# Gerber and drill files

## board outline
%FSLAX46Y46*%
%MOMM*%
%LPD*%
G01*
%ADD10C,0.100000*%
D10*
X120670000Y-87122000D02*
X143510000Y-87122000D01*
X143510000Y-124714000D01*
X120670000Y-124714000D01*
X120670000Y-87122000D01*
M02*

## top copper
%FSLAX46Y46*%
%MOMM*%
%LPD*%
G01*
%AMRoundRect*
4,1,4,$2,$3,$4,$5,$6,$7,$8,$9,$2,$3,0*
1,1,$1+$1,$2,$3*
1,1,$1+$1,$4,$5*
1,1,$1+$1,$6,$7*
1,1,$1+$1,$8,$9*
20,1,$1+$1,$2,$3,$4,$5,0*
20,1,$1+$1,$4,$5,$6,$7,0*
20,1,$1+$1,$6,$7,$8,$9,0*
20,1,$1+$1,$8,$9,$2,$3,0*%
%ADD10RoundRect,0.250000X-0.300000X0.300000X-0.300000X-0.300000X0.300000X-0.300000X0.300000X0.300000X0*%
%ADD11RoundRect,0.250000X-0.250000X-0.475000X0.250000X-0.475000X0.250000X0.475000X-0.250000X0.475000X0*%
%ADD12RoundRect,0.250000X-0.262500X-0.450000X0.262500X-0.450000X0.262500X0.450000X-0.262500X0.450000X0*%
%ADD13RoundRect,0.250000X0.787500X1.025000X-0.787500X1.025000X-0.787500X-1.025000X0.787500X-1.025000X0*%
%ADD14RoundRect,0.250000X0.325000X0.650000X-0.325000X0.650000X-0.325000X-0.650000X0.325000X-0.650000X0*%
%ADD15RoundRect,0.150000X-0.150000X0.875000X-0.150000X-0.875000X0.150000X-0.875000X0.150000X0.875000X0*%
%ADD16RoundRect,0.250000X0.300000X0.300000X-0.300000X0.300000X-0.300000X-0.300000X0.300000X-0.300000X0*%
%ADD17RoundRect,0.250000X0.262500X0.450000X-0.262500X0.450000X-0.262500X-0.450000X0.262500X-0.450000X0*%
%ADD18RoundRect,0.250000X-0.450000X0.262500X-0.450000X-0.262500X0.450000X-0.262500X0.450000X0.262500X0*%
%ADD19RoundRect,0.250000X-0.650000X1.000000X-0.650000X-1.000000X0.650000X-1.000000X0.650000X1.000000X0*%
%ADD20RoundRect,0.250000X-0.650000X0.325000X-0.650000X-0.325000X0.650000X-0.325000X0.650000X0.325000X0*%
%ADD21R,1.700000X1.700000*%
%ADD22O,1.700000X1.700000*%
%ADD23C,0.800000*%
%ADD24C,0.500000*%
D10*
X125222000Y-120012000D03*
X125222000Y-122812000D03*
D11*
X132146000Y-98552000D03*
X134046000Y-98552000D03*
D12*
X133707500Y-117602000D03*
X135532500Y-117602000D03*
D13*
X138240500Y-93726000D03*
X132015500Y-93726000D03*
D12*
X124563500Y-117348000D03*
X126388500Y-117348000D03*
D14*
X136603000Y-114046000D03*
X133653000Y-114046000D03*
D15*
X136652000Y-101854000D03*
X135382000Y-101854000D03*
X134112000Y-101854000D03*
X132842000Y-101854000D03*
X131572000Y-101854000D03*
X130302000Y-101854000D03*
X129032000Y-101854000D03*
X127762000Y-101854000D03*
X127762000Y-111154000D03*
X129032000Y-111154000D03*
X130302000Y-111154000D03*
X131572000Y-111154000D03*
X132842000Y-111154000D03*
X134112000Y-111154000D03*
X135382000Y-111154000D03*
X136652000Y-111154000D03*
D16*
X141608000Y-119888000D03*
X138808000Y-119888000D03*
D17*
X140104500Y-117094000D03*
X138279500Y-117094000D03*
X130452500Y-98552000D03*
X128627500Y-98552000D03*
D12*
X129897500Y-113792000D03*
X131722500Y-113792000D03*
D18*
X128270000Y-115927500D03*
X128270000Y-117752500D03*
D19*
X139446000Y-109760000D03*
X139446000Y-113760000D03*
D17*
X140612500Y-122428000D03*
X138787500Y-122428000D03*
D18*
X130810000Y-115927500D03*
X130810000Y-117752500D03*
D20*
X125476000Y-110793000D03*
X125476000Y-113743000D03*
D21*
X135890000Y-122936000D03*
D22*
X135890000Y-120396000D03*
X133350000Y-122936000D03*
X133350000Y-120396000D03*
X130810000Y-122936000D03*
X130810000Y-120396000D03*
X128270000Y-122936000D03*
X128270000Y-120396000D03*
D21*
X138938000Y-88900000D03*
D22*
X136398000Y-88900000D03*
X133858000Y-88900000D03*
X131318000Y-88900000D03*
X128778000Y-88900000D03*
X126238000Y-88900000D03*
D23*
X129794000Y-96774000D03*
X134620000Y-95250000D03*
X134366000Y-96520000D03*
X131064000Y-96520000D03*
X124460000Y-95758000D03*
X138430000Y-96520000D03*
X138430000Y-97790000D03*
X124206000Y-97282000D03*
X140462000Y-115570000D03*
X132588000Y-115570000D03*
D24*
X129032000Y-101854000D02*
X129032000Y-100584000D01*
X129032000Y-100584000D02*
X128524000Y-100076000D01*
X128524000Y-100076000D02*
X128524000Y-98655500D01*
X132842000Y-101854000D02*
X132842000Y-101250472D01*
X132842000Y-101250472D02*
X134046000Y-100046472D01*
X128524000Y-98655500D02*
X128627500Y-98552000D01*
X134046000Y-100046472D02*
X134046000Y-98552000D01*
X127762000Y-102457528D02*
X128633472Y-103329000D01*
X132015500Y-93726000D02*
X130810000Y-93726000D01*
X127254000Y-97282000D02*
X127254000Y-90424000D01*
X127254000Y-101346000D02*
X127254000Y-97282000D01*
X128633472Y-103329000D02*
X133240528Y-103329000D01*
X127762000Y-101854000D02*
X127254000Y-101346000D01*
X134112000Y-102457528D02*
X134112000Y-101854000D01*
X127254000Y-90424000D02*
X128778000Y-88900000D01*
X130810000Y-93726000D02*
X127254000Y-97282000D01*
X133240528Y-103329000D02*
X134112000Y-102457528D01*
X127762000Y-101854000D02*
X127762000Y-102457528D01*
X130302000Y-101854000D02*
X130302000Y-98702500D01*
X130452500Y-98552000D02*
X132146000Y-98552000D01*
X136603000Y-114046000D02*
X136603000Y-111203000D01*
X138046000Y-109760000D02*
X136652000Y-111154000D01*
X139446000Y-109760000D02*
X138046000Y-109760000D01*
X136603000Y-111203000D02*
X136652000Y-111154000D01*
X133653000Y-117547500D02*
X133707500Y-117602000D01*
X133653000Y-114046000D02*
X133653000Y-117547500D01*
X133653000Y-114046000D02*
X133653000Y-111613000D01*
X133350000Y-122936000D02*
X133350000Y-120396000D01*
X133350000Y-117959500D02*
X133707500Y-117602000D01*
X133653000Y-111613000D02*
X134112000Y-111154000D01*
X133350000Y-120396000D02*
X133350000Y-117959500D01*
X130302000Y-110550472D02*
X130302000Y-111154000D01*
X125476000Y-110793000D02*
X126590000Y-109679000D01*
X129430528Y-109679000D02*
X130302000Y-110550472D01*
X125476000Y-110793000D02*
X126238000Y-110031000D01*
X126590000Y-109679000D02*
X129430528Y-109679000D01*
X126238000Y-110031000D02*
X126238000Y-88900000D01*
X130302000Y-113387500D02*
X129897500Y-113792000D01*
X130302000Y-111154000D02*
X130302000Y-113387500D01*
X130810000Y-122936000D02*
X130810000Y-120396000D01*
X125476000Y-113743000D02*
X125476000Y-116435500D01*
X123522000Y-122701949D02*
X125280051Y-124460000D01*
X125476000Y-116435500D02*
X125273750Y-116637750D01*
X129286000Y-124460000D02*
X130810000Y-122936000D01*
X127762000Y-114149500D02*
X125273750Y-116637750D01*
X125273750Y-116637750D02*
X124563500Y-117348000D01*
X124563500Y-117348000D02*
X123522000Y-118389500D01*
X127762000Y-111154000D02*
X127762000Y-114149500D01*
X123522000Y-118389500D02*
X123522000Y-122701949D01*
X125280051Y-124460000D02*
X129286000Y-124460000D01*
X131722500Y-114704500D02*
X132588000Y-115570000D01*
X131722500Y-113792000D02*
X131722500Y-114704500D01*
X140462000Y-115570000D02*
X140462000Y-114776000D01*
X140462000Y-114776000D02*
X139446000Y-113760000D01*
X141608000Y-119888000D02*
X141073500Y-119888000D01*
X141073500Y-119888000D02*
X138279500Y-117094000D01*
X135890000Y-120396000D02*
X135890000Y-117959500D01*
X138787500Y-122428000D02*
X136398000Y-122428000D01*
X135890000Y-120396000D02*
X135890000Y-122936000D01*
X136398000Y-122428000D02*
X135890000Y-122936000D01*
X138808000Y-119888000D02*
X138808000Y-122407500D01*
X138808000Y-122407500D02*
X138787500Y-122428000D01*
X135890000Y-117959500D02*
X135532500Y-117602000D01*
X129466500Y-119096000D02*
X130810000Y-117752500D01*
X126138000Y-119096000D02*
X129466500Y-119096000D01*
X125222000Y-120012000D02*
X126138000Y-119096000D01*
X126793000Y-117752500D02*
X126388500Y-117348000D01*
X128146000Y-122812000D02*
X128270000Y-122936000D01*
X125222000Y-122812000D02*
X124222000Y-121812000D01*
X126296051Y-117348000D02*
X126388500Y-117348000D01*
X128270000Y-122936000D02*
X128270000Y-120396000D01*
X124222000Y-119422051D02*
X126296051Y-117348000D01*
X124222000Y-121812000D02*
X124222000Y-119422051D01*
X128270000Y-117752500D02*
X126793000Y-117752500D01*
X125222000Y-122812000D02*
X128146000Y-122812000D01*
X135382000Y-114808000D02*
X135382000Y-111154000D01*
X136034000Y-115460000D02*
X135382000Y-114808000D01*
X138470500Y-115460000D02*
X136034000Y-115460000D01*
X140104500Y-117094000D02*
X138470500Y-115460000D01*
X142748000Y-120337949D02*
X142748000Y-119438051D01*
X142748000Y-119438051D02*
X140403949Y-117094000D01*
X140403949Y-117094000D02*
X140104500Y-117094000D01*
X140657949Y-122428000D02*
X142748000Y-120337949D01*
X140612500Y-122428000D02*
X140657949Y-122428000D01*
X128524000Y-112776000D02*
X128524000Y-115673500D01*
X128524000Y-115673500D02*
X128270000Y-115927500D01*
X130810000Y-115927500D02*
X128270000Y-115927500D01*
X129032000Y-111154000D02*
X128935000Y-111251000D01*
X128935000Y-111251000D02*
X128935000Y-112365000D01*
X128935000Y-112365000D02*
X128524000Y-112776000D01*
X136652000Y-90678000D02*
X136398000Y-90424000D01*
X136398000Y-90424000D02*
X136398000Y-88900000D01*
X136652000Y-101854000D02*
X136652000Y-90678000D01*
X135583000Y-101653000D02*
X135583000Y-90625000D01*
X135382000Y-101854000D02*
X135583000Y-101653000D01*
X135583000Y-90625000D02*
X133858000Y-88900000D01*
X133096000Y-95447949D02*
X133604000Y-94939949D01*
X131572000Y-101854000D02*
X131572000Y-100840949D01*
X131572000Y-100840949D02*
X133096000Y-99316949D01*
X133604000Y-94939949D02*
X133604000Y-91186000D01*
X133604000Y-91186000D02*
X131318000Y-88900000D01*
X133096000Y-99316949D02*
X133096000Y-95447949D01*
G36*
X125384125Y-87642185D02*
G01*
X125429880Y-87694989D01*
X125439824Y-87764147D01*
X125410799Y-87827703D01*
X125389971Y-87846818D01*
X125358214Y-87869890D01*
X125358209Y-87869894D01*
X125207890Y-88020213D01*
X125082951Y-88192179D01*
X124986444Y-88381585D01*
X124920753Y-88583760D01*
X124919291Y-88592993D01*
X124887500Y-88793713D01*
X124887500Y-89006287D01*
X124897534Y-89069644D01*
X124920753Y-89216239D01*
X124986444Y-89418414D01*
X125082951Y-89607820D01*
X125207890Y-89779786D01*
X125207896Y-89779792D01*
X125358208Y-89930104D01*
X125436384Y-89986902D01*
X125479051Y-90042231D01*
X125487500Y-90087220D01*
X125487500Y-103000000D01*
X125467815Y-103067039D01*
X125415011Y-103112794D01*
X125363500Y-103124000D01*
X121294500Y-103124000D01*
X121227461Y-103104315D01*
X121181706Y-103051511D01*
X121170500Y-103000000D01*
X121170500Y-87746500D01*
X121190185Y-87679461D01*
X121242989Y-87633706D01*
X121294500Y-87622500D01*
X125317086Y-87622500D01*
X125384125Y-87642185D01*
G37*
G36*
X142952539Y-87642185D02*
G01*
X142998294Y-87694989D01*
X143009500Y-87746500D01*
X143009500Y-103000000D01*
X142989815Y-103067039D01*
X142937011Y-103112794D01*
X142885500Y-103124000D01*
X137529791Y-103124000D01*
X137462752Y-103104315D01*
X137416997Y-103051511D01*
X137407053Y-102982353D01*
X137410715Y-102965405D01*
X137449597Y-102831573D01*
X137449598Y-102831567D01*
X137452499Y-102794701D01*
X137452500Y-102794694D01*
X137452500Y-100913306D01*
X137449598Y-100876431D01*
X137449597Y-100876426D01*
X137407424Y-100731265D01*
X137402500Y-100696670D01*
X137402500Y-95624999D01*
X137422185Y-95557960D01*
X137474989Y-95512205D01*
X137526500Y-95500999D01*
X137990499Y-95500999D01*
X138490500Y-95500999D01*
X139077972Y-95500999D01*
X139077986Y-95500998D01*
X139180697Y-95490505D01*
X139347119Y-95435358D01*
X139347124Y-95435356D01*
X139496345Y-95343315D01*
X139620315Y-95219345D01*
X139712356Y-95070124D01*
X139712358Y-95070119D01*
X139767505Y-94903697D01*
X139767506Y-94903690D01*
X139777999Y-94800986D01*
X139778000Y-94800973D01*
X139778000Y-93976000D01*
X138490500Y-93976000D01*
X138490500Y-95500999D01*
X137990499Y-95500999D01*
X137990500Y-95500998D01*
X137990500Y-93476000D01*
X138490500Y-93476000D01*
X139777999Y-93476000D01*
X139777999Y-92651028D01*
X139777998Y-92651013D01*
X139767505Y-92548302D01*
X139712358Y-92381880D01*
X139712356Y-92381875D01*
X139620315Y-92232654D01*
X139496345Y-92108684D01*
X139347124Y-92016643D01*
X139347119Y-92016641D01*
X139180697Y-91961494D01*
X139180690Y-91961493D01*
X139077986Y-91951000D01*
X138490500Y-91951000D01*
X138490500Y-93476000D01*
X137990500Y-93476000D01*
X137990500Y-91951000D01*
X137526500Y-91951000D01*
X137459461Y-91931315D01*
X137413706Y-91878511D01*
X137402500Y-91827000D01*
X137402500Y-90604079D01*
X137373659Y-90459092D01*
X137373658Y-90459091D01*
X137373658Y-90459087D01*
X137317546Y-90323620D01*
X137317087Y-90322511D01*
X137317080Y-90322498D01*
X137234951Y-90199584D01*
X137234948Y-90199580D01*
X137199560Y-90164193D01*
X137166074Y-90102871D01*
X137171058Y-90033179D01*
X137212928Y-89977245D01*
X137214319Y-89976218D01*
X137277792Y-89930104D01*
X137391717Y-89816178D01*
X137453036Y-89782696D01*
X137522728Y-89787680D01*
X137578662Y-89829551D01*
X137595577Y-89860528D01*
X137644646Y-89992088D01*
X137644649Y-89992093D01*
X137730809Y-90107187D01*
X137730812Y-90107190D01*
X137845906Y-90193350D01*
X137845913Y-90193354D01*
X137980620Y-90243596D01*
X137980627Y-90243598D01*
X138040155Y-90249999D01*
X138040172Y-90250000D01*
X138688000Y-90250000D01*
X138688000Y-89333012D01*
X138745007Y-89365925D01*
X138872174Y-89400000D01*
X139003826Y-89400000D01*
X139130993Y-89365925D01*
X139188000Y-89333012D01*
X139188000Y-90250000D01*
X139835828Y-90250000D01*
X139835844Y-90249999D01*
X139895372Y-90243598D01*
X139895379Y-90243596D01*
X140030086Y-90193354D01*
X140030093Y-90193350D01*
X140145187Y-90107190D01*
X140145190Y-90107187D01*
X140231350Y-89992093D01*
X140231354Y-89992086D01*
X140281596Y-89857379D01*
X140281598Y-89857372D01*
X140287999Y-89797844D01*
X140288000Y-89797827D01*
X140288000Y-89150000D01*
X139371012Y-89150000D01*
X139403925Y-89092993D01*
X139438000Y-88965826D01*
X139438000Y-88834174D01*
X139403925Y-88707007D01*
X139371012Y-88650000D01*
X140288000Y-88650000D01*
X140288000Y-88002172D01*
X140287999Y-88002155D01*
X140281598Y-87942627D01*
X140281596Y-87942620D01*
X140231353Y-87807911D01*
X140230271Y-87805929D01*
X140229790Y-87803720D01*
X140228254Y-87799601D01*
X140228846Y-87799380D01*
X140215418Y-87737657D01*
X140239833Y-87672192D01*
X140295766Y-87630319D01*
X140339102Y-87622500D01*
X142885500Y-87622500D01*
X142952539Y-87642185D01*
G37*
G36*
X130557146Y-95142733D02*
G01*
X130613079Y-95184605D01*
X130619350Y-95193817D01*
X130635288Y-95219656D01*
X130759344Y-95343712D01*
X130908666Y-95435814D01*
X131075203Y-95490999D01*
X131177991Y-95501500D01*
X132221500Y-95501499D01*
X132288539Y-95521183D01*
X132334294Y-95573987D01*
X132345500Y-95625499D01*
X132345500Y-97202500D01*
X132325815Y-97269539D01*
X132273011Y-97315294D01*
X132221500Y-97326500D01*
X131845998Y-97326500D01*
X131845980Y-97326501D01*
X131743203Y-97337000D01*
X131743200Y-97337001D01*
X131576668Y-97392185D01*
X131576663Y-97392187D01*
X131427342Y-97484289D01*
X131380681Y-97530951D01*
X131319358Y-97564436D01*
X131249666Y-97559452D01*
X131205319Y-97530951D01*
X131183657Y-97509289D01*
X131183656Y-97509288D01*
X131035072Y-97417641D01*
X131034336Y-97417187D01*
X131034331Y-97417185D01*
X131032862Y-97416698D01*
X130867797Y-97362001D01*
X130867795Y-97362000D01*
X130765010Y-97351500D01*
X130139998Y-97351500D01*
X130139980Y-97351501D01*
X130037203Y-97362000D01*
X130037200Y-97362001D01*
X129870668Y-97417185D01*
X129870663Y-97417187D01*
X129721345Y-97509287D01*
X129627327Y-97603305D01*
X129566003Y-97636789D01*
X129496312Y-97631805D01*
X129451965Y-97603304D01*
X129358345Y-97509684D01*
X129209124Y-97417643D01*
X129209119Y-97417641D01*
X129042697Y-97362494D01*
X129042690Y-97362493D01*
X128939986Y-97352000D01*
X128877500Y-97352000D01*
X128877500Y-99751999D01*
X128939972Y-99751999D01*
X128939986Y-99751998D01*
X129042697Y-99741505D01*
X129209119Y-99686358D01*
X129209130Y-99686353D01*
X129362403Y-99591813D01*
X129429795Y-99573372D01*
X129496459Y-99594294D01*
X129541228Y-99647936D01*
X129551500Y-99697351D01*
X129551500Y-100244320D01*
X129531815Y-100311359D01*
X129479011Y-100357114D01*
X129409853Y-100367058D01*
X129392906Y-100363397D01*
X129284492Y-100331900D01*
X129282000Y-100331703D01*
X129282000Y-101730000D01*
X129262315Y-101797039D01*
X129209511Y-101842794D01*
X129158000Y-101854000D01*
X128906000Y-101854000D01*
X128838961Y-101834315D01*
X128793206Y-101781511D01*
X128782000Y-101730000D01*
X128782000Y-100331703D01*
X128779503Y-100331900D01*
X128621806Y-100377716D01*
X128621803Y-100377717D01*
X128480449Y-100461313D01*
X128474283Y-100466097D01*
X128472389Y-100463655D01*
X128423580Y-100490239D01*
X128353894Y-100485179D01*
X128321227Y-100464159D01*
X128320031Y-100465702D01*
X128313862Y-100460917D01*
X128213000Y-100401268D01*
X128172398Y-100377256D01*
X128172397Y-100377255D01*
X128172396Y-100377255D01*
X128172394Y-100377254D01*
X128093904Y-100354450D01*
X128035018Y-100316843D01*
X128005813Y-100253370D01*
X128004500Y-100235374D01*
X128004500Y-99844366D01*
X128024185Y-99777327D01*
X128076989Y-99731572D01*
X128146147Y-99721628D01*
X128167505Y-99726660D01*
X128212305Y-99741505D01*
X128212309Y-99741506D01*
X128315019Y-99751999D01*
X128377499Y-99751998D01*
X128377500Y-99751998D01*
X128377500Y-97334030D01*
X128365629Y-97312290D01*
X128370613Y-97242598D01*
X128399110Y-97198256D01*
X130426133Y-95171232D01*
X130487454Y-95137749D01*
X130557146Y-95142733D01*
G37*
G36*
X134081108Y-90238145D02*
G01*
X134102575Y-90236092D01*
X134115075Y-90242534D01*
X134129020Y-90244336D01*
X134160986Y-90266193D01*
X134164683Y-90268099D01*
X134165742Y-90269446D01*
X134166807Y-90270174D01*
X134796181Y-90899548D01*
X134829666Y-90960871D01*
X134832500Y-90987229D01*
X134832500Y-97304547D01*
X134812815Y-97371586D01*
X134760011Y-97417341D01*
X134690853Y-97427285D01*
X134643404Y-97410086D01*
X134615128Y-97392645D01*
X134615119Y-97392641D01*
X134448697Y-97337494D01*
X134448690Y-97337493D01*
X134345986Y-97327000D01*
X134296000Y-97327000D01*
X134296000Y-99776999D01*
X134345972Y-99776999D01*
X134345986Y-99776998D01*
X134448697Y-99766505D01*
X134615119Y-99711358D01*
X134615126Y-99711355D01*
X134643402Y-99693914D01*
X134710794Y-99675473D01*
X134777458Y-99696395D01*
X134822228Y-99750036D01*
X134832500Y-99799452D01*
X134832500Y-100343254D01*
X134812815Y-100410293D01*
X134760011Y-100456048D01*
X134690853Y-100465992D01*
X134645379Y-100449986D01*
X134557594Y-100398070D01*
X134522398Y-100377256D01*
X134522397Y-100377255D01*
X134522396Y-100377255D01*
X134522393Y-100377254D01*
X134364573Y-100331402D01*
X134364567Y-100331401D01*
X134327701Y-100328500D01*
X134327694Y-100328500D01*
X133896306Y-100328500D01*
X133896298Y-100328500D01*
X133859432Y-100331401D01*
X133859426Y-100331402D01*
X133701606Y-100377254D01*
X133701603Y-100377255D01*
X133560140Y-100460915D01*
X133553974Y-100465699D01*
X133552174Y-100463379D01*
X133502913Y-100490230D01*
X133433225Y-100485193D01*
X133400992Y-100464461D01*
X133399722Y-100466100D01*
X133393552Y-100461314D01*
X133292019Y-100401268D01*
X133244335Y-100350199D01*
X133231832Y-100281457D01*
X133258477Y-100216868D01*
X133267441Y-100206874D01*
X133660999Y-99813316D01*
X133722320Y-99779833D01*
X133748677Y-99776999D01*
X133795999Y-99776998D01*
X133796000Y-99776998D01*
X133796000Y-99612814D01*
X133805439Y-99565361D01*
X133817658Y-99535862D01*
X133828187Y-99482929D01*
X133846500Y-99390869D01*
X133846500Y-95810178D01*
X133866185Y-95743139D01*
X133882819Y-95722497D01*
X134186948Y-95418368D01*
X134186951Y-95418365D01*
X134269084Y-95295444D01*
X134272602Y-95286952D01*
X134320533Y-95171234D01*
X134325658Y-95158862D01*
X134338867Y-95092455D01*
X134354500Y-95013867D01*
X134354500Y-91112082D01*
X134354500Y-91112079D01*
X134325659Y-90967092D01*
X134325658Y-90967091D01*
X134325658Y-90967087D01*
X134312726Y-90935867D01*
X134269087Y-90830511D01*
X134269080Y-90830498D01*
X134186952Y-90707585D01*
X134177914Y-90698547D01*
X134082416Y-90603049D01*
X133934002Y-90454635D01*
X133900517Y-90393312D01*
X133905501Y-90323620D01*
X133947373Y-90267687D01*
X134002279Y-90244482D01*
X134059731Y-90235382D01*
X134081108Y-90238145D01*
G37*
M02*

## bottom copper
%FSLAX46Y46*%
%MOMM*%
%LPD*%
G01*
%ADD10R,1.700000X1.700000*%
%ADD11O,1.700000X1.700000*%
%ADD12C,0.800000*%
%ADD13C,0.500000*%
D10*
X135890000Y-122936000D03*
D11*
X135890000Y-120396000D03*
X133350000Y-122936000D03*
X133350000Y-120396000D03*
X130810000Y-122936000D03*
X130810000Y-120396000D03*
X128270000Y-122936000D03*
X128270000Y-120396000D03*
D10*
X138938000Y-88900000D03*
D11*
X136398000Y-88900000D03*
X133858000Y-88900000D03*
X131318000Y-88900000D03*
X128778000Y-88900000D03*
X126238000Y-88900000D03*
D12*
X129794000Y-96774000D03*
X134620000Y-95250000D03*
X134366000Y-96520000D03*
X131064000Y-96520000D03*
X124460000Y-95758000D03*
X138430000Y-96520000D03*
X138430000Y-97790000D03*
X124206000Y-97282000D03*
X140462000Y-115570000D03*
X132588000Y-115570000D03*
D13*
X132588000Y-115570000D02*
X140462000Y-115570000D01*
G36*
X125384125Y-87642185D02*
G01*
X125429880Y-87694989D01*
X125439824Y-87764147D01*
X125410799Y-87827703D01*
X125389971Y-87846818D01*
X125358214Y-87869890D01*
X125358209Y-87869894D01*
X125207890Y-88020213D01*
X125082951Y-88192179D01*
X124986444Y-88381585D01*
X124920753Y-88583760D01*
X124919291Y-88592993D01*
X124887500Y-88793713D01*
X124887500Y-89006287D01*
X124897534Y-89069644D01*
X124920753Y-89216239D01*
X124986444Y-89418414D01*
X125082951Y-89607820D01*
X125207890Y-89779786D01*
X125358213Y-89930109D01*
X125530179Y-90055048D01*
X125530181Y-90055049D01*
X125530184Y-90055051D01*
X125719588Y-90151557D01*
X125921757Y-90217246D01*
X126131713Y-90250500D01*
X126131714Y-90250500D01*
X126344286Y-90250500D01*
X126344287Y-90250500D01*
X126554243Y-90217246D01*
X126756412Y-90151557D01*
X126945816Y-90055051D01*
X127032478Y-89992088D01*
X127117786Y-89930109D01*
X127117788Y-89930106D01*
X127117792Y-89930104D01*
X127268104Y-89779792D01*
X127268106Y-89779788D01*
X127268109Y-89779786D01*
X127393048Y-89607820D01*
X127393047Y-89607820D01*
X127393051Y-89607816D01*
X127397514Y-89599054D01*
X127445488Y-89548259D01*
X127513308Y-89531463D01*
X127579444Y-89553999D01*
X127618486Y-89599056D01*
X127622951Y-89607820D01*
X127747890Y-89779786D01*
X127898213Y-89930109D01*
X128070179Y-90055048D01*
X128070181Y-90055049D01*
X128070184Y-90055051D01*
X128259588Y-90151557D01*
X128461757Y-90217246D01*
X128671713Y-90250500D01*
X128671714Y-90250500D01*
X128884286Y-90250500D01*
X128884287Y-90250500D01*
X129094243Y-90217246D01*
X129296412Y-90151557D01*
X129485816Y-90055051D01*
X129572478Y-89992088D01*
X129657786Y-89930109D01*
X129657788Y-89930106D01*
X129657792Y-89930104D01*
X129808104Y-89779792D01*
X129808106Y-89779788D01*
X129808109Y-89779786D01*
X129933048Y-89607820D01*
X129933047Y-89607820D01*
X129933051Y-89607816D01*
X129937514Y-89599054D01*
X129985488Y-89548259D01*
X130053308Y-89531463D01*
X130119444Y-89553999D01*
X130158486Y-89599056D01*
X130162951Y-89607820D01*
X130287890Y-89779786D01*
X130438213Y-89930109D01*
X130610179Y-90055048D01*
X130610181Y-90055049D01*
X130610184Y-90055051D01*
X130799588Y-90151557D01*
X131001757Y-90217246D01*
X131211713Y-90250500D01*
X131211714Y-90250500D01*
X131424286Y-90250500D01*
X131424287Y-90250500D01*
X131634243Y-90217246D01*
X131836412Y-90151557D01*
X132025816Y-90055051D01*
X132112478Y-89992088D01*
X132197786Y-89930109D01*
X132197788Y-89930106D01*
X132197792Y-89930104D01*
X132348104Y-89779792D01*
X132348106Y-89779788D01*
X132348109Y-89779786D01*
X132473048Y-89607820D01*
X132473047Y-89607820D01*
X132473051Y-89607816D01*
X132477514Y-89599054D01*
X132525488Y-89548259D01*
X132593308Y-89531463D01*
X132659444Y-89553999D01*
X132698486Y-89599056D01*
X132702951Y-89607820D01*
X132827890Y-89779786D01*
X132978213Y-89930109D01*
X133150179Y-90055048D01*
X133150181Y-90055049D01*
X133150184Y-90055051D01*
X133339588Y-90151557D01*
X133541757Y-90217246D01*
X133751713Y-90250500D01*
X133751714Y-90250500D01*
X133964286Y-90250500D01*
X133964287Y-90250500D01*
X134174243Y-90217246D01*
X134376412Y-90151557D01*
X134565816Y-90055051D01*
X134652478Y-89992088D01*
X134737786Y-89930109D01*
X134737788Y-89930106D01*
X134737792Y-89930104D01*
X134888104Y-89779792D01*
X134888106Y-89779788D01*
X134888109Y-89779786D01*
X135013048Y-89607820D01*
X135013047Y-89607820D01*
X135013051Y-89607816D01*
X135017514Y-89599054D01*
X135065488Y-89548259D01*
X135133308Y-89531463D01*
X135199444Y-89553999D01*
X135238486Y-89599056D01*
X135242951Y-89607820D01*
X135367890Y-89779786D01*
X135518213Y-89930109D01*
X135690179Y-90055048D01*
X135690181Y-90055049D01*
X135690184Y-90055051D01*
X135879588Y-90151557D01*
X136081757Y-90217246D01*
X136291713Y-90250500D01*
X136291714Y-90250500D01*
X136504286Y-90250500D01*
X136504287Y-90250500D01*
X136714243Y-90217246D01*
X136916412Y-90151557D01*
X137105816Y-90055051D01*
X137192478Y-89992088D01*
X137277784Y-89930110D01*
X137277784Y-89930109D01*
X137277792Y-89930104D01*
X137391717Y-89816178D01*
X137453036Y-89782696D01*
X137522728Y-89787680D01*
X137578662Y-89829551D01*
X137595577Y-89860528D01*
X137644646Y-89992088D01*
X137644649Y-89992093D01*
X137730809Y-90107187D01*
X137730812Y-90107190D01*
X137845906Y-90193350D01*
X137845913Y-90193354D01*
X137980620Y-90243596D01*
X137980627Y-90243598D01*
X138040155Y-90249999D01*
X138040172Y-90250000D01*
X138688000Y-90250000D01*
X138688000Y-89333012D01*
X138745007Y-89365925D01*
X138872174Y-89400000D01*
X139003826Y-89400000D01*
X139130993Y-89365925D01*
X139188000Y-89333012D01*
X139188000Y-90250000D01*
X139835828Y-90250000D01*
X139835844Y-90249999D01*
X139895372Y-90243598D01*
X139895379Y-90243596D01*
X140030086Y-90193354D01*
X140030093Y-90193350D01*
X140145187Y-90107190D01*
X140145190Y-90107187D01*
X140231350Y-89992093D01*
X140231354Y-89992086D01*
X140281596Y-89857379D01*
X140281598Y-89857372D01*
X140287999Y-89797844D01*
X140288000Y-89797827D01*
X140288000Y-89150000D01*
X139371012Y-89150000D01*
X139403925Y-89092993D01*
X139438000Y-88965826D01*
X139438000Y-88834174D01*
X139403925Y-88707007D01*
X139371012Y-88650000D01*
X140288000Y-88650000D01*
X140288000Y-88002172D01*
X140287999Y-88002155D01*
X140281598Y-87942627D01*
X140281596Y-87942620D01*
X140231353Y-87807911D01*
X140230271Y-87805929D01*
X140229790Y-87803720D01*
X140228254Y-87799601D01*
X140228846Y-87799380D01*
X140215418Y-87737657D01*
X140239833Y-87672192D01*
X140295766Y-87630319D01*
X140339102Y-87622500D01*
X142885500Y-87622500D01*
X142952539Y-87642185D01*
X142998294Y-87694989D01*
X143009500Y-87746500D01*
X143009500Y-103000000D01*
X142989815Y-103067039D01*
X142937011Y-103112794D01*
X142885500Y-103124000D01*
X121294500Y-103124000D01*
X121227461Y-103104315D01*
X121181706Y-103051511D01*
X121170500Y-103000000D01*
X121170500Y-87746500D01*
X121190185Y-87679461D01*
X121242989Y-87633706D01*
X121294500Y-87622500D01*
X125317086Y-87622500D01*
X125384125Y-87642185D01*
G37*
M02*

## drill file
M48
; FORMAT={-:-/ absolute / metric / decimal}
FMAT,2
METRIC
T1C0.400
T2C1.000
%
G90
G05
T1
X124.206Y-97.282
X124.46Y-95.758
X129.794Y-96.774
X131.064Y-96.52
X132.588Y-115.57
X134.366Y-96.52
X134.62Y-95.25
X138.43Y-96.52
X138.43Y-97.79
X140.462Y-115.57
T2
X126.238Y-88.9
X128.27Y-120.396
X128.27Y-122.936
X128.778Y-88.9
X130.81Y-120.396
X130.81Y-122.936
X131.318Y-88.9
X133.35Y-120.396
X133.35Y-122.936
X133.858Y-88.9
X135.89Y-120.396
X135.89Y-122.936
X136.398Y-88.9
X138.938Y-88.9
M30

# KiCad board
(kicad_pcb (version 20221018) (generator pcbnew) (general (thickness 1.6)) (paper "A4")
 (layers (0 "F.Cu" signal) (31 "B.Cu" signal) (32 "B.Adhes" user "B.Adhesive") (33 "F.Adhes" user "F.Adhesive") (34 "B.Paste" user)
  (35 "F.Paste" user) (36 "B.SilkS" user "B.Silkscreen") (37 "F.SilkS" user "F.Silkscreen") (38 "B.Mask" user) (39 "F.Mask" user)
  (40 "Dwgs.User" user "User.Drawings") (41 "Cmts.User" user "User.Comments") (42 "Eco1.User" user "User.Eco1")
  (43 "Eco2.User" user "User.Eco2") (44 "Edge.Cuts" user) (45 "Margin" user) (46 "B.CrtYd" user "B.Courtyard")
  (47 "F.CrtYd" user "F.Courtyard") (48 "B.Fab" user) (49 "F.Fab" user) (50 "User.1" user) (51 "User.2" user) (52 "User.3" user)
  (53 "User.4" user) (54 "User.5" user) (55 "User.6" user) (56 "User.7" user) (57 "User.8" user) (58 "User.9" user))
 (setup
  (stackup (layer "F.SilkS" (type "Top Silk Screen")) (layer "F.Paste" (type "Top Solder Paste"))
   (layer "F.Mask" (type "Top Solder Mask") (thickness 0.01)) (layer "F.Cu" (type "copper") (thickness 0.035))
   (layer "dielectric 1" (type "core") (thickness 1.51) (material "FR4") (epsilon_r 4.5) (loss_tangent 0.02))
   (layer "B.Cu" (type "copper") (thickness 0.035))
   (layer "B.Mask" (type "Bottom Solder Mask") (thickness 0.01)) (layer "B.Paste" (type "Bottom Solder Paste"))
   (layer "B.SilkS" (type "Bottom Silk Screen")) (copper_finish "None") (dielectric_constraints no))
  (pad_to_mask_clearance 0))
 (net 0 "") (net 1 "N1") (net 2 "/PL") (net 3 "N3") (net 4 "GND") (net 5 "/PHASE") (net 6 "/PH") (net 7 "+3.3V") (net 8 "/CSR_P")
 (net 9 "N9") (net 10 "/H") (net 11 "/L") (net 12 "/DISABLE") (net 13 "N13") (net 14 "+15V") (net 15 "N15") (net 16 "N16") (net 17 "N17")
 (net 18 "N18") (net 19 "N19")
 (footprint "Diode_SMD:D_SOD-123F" (layer "F.Cu") (at 125.222 121.412 -90)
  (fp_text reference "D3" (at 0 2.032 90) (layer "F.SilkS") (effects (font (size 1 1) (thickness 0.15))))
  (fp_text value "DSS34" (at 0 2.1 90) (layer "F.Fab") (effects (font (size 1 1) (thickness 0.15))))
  (pad "1" smd roundrect (at -1.4 0 270) (size 1.1 1.1) (layers "F.Cu" "F.Paste" "F.Mask") (roundrect_rratio 0.2272727273) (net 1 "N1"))
  (pad "2" smd roundrect (at 1.4 0 270) (size 1.1 1.1) (layers "F.Cu" "F.Paste" "F.Mask") (roundrect_rratio 0.2272727273) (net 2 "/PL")))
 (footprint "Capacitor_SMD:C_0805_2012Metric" (layer "F.Cu") (at 133.096 98.552)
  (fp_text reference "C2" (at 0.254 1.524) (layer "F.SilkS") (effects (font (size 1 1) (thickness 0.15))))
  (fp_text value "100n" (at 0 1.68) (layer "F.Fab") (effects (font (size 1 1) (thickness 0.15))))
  (pad "1" smd roundrect (at -0.95 0) (size 1 1.45) (layers "F.Cu" "F.Paste" "F.Mask") (roundrect_rratio 0.25) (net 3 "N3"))
  (pad "2" smd roundrect (at 0.95 0) (size 1 1.45) (layers "F.Cu" "F.Paste" "F.Mask") (roundrect_rratio 0.25) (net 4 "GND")))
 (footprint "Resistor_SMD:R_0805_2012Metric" (layer "F.Cu") (at 134.62 117.602)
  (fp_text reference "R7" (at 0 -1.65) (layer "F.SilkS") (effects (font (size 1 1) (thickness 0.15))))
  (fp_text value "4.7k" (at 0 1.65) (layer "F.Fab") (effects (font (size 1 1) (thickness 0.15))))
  (pad "1" smd roundrect (at -0.9125 0) (size 1.025 1.4) (layers "F.Cu" "F.Paste" "F.Mask") (roundrect_rratio 0.243902) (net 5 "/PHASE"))
  (pad "2" smd roundrect (at 0.9125 0) (size 1.025 1.4) (layers "F.Cu" "F.Paste" "F.Mask") (roundrect_rratio 0.243902) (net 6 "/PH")))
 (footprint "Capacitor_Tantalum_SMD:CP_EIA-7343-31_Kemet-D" (layer "F.Cu") (at 135.128 93.726 180)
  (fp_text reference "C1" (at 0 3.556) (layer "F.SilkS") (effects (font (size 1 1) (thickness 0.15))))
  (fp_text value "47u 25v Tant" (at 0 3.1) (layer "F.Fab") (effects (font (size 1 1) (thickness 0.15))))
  (pad "1" smd roundrect (at -3.1125 0 180) (size 2.075 2.55) (layers "F.Cu" "F.Paste" "F.Mask") (roundrect_rratio 0.120482) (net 4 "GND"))
  (pad "2" smd roundrect (at 3.1125 0 180) (size 2.075 2.55) (layers "F.Cu" "F.Paste" "F.Mask") (roundrect_rratio 0.120482) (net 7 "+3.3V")))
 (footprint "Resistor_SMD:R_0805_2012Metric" (layer "F.Cu") (at 125.476 117.348)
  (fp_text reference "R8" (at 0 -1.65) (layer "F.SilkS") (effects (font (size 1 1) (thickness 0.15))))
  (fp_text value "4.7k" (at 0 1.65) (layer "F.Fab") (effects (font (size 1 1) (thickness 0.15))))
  (pad "1" smd roundrect (at -0.9125 0) (size 1.025 1.4) (layers "F.Cu" "F.Paste" "F.Mask") (roundrect_rratio 0.243902) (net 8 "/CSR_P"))
  (pad "2" smd roundrect (at 0.9125 0) (size 1.025 1.4) (layers "F.Cu" "F.Paste" "F.Mask") (roundrect_rratio 0.243902) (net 2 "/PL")))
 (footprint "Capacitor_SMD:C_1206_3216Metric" (layer "F.Cu") (at 135.128 114.046 180)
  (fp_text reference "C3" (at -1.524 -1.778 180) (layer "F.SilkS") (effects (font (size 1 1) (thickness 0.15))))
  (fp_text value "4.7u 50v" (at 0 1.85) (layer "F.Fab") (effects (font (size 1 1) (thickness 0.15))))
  (pad "1" smd roundrect (at -1.475 0 180) (size 1.15 1.8) (layers "F.Cu" "F.Paste" "F.Mask") (roundrect_rratio 0.217391) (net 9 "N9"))
  (pad "2" smd roundrect (at 1.475 0 180) (size 1.15 1.8) (layers "F.Cu" "F.Paste" "F.Mask") (roundrect_rratio 0.217391) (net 5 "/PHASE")))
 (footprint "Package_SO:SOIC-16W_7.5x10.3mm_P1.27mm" (layer "F.Cu") (at 132.207 106.504 -90)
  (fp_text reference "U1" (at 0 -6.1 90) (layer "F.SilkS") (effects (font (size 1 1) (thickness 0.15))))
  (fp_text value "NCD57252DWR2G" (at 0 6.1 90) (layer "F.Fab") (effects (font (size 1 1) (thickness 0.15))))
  (pad "1" smd roundrect (at -4.65 -4.445 270) (size 2.05 0.6) (layers "F.Cu" "F.Paste" "F.Mask") (roundrect_rratio 0.25) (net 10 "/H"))
  (pad "2" smd roundrect (at -4.65 -3.175 270) (size 2.05 0.6) (layers "F.Cu" "F.Paste" "F.Mask") (roundrect_rratio 0.25) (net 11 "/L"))
  (pad "3" smd roundrect (at -4.65 -1.905 270) (size 2.05 0.6) (layers "F.Cu" "F.Paste" "F.Mask") (roundrect_rratio 0.25) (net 7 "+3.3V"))
  (pad "4" smd roundrect (at -4.65 -0.635 270) (size 2.05 0.6) (layers "F.Cu" "F.Paste" "F.Mask") (roundrect_rratio 0.25) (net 4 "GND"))
  (pad "5" smd roundrect (at -4.65 0.635 270) (size 2.05 0.6) (layers "F.Cu" "F.Paste" "F.Mask") (roundrect_rratio 0.25) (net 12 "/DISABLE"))
  (pad "6" smd roundrect (at -4.65 1.905 270) (size 2.05 0.6) (layers "F.Cu" "F.Paste" "F.Mask") (roundrect_rratio 0.25) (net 3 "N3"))
  (pad "7" smd roundrect (at -4.65 3.175 270) (size 2.05 0.6) (layers "F.Cu" "F.Paste" "F.Mask") (roundrect_rratio 0.25) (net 4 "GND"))
  (pad "8" smd roundrect (at -4.65 4.445 270) (size 2.05 0.6) (layers "F.Cu" "F.Paste" "F.Mask") (roundrect_rratio 0.25) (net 7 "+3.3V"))
  (pad "9" smd roundrect (at 4.65 4.445 270) (size 2.05 0.6) (layers "F.Cu" "F.Paste" "F.Mask") (roundrect_rratio 0.25) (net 8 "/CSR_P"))
  (pad "10" smd roundrect (at 4.65 3.175 270) (size 2.05 0.6) (layers "F.Cu" "F.Paste" "F.Mask") (roundrect_rratio 0.25) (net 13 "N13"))
  (pad "11" smd roundrect (at 4.65 1.905 270) (size 2.05 0.6) (layers "F.Cu" "F.Paste" "F.Mask") (roundrect_rratio 0.25) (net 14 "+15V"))
  (pad "12" smd roundrect (at 4.65 0.635 270) (size 2.05 0.6) (layers "F.Cu" "F.Paste" "F.Mask") (roundrect_rratio 0.25) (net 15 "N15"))
  (pad "13" smd roundrect (at 4.65 -0.635 270) (size 2.05 0.6) (layers "F.Cu" "F.Paste" "F.Mask") (roundrect_rratio 0.25) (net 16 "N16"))
  (pad "14" smd roundrect (at 4.65 -1.905 270) (size 2.05 0.6) (layers "F.Cu" "F.Paste" "F.Mask") (roundrect_rratio 0.25) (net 5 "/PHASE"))
  (pad "15" smd roundrect (at 4.65 -3.175 270) (size 2.05 0.6) (layers "F.Cu" "F.Paste" "F.Mask") (roundrect_rratio 0.25) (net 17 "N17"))
  (pad "16" smd roundrect (at 4.65 -4.445 270) (size 2.05 0.6) (layers "F.Cu" "F.Paste" "F.Mask") (roundrect_rratio 0.25) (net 9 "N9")))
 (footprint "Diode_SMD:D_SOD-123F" (layer "F.Cu") (at 140.208 119.888 180)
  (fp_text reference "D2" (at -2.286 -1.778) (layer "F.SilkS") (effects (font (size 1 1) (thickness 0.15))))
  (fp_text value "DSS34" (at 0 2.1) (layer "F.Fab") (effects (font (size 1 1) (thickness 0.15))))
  (pad "1" smd roundrect (at -1.4 0 180) (size 1.1 1.1) (layers "F.Cu" "F.Paste" "F.Mask") (roundrect_rratio 0.2272727273) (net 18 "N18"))
  (pad "2" smd roundrect (at 1.4 0 180) (size 1.1 1.1) (layers "F.Cu" "F.Paste" "F.Mask") (roundrect_rratio 0.2272727273) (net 6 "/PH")))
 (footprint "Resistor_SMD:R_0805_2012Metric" (layer "F.Cu") (at 139.192 117.094 180)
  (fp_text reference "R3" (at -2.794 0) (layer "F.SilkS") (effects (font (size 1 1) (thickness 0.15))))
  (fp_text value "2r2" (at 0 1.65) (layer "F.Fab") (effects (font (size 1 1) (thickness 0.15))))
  (pad "1" smd roundrect (at -0.9125 0 180) (size 1.025 1.4) (layers "F.Cu" "F.Paste" "F.Mask") (roundrect_rratio 0.243902) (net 17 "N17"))
  (pad "2" smd roundrect (at 0.9125 0 180) (size 1.025 1.4) (layers "F.Cu" "F.Paste" "F.Mask") (roundrect_rratio 0.243902) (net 18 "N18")))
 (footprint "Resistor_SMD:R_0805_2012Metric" (layer "F.Cu") (at 129.54 98.552 180)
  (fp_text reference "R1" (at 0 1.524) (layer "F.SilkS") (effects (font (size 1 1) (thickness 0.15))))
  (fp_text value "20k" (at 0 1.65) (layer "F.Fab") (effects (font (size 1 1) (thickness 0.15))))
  (pad "1" smd roundrect (at -0.9125 0 180) (size 1.025 1.4) (layers "F.Cu" "F.Paste" "F.Mask") (roundrect_rratio 0.243902) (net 3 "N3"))
  (pad "2" smd roundrect (at 0.9125 0 180) (size 1.025 1.4) (layers "F.Cu" "F.Paste" "F.Mask") (roundrect_rratio 0.243902) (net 4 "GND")))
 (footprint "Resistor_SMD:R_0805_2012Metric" (layer "F.Cu") (at 130.81 113.792)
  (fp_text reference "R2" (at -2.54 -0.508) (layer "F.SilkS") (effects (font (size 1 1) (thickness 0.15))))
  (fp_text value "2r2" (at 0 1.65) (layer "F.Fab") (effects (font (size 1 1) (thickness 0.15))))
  (pad "1" smd roundrect (at -0.9125 0) (size 1.025 1.4) (layers "F.Cu" "F.Paste" "F.Mask") (roundrect_rratio 0.243902) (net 14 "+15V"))
  (pad "2" smd roundrect (at 0.9125 0) (size 1.025 1.4) (layers "F.Cu" "F.Paste" "F.Mask") (roundrect_rratio 0.243902) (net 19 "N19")))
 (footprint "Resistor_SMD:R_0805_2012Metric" (layer "F.Cu") (at 128.27 116.84 -90)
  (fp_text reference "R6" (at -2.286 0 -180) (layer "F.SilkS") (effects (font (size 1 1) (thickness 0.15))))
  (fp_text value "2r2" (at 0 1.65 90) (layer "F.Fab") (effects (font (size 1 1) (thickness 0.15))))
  (pad "1" smd roundrect (at -0.9125 0 270) (size 1.025 1.4) (layers "F.Cu" "F.Paste" "F.Mask") (roundrect_rratio 0.243902) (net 13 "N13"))
  (pad "2" smd roundrect (at 0.9125 0 270) (size 1.025 1.4) (layers "F.Cu" "F.Paste" "F.Mask") (roundrect_rratio 0.243902) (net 2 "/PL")))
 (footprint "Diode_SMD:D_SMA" (layer "F.Cu") (at 139.446 111.76 -90)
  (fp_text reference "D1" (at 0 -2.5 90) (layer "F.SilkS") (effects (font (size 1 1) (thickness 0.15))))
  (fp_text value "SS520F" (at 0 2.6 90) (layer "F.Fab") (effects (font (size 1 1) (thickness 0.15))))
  (pad "1" smd roundrect (at -2 0 270) (size 2.5 1.8) (layers "F.Cu" "F.Paste" "F.Mask") (roundrect_rratio 0.1388888889) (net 9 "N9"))
  (pad "2" smd roundrect (at 2 0 270) (size 2.5 1.8) (layers "F.Cu" "F.Paste" "F.Mask") (roundrect_rratio 0.1388888889) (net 19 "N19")))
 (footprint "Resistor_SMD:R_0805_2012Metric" (layer "F.Cu") (at 139.7 122.428 180)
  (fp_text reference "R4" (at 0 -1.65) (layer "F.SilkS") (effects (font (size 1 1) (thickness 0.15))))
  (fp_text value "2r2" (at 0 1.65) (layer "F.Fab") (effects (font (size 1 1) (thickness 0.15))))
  (pad "1" smd roundrect (at -0.9125 0 180) (size 1.025 1.4) (layers "F.Cu" "F.Paste" "F.Mask") (roundrect_rratio 0.243902) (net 17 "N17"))
  (pad "2" smd roundrect (at 0.9125 0 180) (size 1.025 1.4) (layers "F.Cu" "F.Paste" "F.Mask") (roundrect_rratio 0.243902) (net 6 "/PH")))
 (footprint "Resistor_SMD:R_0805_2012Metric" (layer "F.Cu") (at 130.81 116.84 -90)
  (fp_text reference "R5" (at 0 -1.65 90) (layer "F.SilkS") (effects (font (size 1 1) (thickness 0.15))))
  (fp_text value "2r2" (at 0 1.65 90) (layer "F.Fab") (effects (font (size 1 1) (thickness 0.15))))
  (pad "1" smd roundrect (at -0.9125 0 270) (size 1.025 1.4) (layers "F.Cu" "F.Paste" "F.Mask") (roundrect_rratio 0.243902) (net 13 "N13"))
  (pad "2" smd roundrect (at 0.9125 0 270) (size 1.025 1.4) (layers "F.Cu" "F.Paste" "F.Mask") (roundrect_rratio 0.243902) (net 1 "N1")))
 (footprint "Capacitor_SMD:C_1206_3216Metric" (layer "F.Cu") (at 125.476 112.268 -90)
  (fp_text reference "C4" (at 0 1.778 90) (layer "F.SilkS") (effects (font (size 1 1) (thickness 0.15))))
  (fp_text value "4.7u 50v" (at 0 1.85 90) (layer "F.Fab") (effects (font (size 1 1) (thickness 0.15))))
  (pad "1" smd roundrect (at -1.475 0 270) (size 1.15 1.8) (layers "F.Cu" "F.Paste" "F.Mask") (roundrect_rratio 0.217391) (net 14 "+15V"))
  (pad "2" smd roundrect (at 1.475 0 270) (size 1.15 1.8) (layers "F.Cu" "F.Paste" "F.Mask") (roundrect_rratio 0.217391) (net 8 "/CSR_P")))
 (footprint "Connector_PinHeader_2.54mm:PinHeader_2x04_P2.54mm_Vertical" (layer "B.Cu") (at 135.89 122.936 90)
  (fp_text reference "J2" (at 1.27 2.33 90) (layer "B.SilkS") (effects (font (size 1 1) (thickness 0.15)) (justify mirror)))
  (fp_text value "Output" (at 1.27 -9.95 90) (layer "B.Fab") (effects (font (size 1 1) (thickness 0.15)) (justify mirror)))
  (pad "1" thru_hole rect (at 0 0 90) (size 1.7 1.7) (drill 1) (layers "*.Cu" "*.Mask") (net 6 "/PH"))
  (pad "2" thru_hole oval (at 2.54 0 90) (size 1.7 1.7) (drill 1) (layers "*.Cu" "*.Mask") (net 6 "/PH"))
  (pad "3" thru_hole oval (at 0 -2.54 90) (size 1.7 1.7) (drill 1) (layers "*.Cu" "*.Mask") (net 5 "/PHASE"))
  (pad "4" thru_hole oval (at 2.54 -2.54 90) (size 1.7 1.7) (drill 1) (layers "*.Cu" "*.Mask") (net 5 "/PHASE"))
  (pad "5" thru_hole oval (at 0 -5.08 90) (size 1.7 1.7) (drill 1) (layers "*.Cu" "*.Mask") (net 8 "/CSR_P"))
  (pad "6" thru_hole oval (at 2.54 -5.08 90) (size 1.7 1.7) (drill 1) (layers "*.Cu" "*.Mask") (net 8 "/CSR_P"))
  (pad "7" thru_hole oval (at 0 -7.62 90) (size 1.7 1.7) (drill 1) (layers "*.Cu" "*.Mask") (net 2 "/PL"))
  (pad "8" thru_hole oval (at 2.54 -7.62 90) (size 1.7 1.7) (drill 1) (layers "*.Cu" "*.Mask") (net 2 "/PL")))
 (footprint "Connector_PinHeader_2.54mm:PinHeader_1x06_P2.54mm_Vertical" (layer "B.Cu") (at 138.938 88.9 90)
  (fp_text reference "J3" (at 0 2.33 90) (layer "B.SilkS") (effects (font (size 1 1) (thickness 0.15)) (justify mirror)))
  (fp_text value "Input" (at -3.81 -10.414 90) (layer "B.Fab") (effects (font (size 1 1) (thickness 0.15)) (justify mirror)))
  (pad "1" thru_hole rect (at 0 0 90) (size 1.7 1.7) (drill 1) (layers "*.Cu" "*.Mask") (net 4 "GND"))
  (pad "2" thru_hole oval (at 0 -2.54 90) (size 1.7 1.7) (drill 1) (layers "*.Cu" "*.Mask") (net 10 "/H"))
  (pad "3" thru_hole oval (at 0 -5.08 90) (size 1.7 1.7) (drill 1) (layers "*.Cu" "*.Mask") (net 11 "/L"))
  (pad "4" thru_hole oval (at 0 -7.62 90) (size 1.7 1.7) (drill 1) (layers "*.Cu" "*.Mask") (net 12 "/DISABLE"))
  (pad "5" thru_hole oval (at 0 -10.16 90) (size 1.7 1.7) (drill 1) (layers "*.Cu" "*.Mask") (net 7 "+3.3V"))
  (pad "6" thru_hole oval (at 0 -12.7 90) (size 1.7 1.7) (drill 1) (layers "*.Cu" "*.Mask") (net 14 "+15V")))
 (gr_rect (start 120.67 87.122) (end 143.51 124.714) (stroke (width 0.1) (type default)) (fill none) (layer "Edge.Cuts"))
 (segment (start 129.032 101.854) (end 129.032 100.584) (width 0.5) (layer "F.Cu") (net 4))
 (segment (start 129.032 100.584) (end 128.524 100.076) (width 0.5) (layer "F.Cu") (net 4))
 (segment (start 128.524 100.076) (end 128.524 98.6555) (width 0.5) (layer "F.Cu") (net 4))
 (segment (start 132.842 101.854) (end 132.842 101.250472) (width 0.5) (layer "F.Cu") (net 4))
 (segment (start 132.842 101.250472) (end 134.046 100.046472) (width 0.5) (layer "F.Cu") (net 4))
 (segment (start 128.524 98.6555) (end 128.6275 98.552) (width 0.5) (layer "F.Cu") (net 4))
 (segment (start 134.046 100.046472) (end 134.046 98.552) (width 0.5) (layer "F.Cu") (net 4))
 (via (at 129.794 96.774) (size 0.8) (drill 0.4) (layers "F.Cu" "B.Cu") (free) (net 4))
 (via (at 134.62 95.25) (size 0.8) (drill 0.4) (layers "F.Cu" "B.Cu") (free) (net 4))
 (via (at 134.366 96.52) (size 0.8) (drill 0.4) (layers "F.Cu" "B.Cu") (free) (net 4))
 (via (at 131.064 96.52) (size 0.8) (drill 0.4) (layers "F.Cu" "B.Cu") (free) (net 4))
 (via (at 124.46 95.758) (size 0.8) (drill 0.4) (layers "F.Cu" "B.Cu") (free) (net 4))
 (via (at 138.43 96.52) (size 0.8) (drill 0.4) (layers "F.Cu" "B.Cu") (free) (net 4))
 (via (at 138.43 97.79) (size 0.8) (drill 0.4) (layers "F.Cu" "B.Cu") (free) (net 4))
 (via (at 124.206 97.282) (size 0.8) (drill 0.4) (layers "F.Cu" "B.Cu") (free) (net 4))
 (segment (start 127.762 102.457528) (end 128.633472 103.329) (width 0.5) (layer "F.Cu") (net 7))
 (segment (start 132.0155 93.726) (end 130.81 93.726) (width 0.5) (layer "F.Cu") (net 7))
 (segment (start 127.254 97.282) (end 127.254 90.424) (width 0.5) (layer "F.Cu") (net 7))
 (segment (start 127.254 101.346) (end 127.254 97.282) (width 0.5) (layer "F.Cu") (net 7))
 (segment (start 128.633472 103.329) (end 133.240528 103.329) (width 0.5) (layer "F.Cu") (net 7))
 (segment (start 127.762 101.854) (end 127.254 101.346) (width 0.5) (layer "F.Cu") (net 7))
 (segment (start 134.112 102.457528) (end 134.112 101.854) (width 0.5) (layer "F.Cu") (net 7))
 (segment (start 127.254 90.424) (end 128.778 88.9) (width 0.5) (layer "F.Cu") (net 7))
 (segment (start 130.81 93.726) (end 127.254 97.282) (width 0.5) (layer "F.Cu") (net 7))
 (segment (start 133.240528 103.329) (end 134.112 102.457528) (width 0.5) (layer "F.Cu") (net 7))
 (segment (start 127.762 101.854) (end 127.762 102.457528) (width 0.5) (layer "F.Cu") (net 7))
 (segment (start 130.302 101.854) (end 130.302 98.7025) (width 0.5) (layer "F.Cu") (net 3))
 (segment (start 130.4525 98.552) (end 132.146 98.552) (width 0.5) (layer "F.Cu") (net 3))
 (segment (start 136.603 114.046) (end 136.603 111.203) (width 0.5) (layer "F.Cu") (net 9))
 (segment (start 138.046 109.76) (end 136.652 111.154) (width 0.5) (layer "F.Cu") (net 9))
 (segment (start 139.446 109.76) (end 138.046 109.76) (width 0.5) (layer "F.Cu") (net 9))
 (segment (start 136.603 111.203) (end 136.652 111.154) (width 0.5) (layer "F.Cu") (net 9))
 (segment (start 133.653 117.5475) (end 133.7075 117.602) (width 0.5) (layer "F.Cu") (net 5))
 (segment (start 133.653 114.046) (end 133.653 117.5475) (width 0.5) (layer "F.Cu") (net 5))
 (segment (start 133.653 114.046) (end 133.653 111.613) (width 0.5) (layer "F.Cu") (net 5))
 (segment (start 133.35 122.936) (end 133.35 120.396) (width 0.5) (layer "F.Cu") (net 5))
 (segment (start 133.35 117.9595) (end 133.7075 117.602) (width 0.5) (layer "F.Cu") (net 5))
 (segment (start 133.653 111.613) (end 134.112 111.154) (width 0.5) (layer "F.Cu") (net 5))
 (segment (start 133.35 120.396) (end 133.35 117.9595) (width 0.5) (layer "F.Cu") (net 5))
 (segment (start 130.302 110.550472) (end 130.302 111.154) (width 0.5) (layer "F.Cu") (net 14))
 (segment (start 125.476 110.793) (end 126.59 109.679) (width 0.5) (layer "F.Cu") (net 14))
 (segment (start 129.430528 109.679) (end 130.302 110.550472) (width 0.5) (layer "F.Cu") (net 14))
 (segment (start 125.476 110.793) (end 126.238 110.031) (width 0.5) (layer "F.Cu") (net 14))
 (segment (start 126.59 109.679) (end 129.430528 109.679) (width 0.5) (layer "F.Cu") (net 14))
 (segment (start 126.238 110.031) (end 126.238 88.9) (width 0.5) (layer "F.Cu") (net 14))
 (segment (start 130.302 113.3875) (end 129.8975 113.792) (width 0.5) (layer "F.Cu") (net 14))
 (segment (start 130.302 111.154) (end 130.302 113.3875) (width 0.5) (layer "F.Cu") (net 14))
 (segment (start 130.81 122.936) (end 130.81 120.396) (width 0.5) (layer "F.Cu") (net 8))
 (segment (start 125.476 113.743) (end 125.476 116.4355) (width 0.5) (layer "F.Cu") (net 8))
 (segment (start 123.522 122.701949) (end 125.280051 124.46) (width 0.5) (layer "F.Cu") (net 8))
 (segment (start 125.476 116.4355) (end 125.27375 116.63775) (width 0.5) (layer "F.Cu") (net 8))
 (segment (start 129.286 124.46) (end 130.81 122.936) (width 0.5) (layer "F.Cu") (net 8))
 (segment (start 127.762 114.1495) (end 125.27375 116.63775) (width 0.5) (layer "F.Cu") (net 8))
 (segment (start 125.27375 116.63775) (end 124.5635 117.348) (width 0.5) (layer "F.Cu") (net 8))
 (segment (start 124.5635 117.348) (end 123.522 118.3895) (width 0.5) (layer "F.Cu") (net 8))
 (segment (start 127.762 111.154) (end 127.762 114.1495) (width 0.5) (layer "F.Cu") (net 8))
 (segment (start 123.522 118.3895) (end 123.522 122.701949) (width 0.5) (layer "F.Cu") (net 8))
 (segment (start 125.280051 124.46) (end 129.286 124.46) (width 0.5) (layer "F.Cu") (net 8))
 (segment (start 131.7225 114.7045) (end 132.588 115.57) (width 0.5) (layer "F.Cu") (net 19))
 (segment (start 131.7225 113.792) (end 131.7225 114.7045) (width 0.5) (layer "F.Cu") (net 19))
 (segment (start 140.462 115.57) (end 140.462 114.776) (width 0.5) (layer "F.Cu") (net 19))
 (segment (start 140.462 114.776) (end 139.446 113.76) (width 0.5) (layer "F.Cu") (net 19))
 (via (at 140.462 115.57) (size 0.8) (drill 0.4) (layers "F.Cu" "B.Cu") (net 19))
 (via (at 132.588 115.57) (size 0.8) (drill 0.4) (layers "F.Cu" "B.Cu") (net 19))
 (segment (start 132.588 115.57) (end 140.462 115.57) (width 0.5) (layer "B.Cu") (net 19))
 (segment (start 141.608 119.888) (end 141.0735 119.888) (width 0.5) (layer "F.Cu") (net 18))
 (segment (start 141.0735 119.888) (end 138.2795 117.094) (width 0.5) (layer "F.Cu") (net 18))
 (segment (start 135.89 120.396) (end 135.89 117.9595) (width 0.5) (layer "F.Cu") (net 6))
 (segment (start 138.7875 122.428) (end 136.398 122.428) (width 0.5) (layer "F.Cu") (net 6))
 (segment (start 135.89 120.396) (end 135.89 122.936) (width 0.5) (layer "F.Cu") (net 6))
 (segment (start 136.398 122.428) (end 135.89 122.936) (width 0.5) (layer "F.Cu") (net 6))
 (segment (start 138.808 119.888) (end 138.808 122.4075) (width 0.5) (layer "F.Cu") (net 6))
 (segment (start 138.808 122.4075) (end 138.7875 122.428) (width 0.5) (layer "F.Cu") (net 6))
 (segment (start 135.89 117.9595) (end 135.5325 117.602) (width 0.5) (layer "F.Cu") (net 6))
 (segment (start 129.4665 119.096) (end 130.81 117.7525) (width 0.5) (layer "F.Cu") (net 1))
 (segment (start 126.138 119.096) (end 129.4665 119.096) (width 0.5) (layer "F.Cu") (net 1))
 (segment (start 125.222 120.012) (end 126.138 119.096) (width 0.5) (layer "F.Cu") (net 1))
 (segment (start 126.793 117.7525) (end 126.3885 117.348) (width 0.5) (layer "F.Cu") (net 2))
 (segment (start 128.146 122.812) (end 128.27 122.936) (width 0.5) (layer "F.Cu") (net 2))
 (segment (start 125.222 122.812) (end 124.222 121.812) (width 0.5) (layer "F.Cu") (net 2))
 (segment (start 126.296051 117.348) (end 126.3885 117.348) (width 0.5) (layer "F.Cu") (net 2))
 (segment (start 128.27 122.936) (end 128.27 120.396) (width 0.5) (layer "F.Cu") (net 2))
 (segment (start 124.222 119.422051) (end 126.296051 117.348) (width 0.5) (layer "F.Cu") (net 2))
 (segment (start 124.222 121.812) (end 124.222 119.422051) (width 0.5) (layer "F.Cu") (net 2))
 (segment (start 128.27 117.7525) (end 126.793 117.7525) (width 0.5) (layer "F.Cu") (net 2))
 (segment (start 125.222 122.812) (end 128.146 122.812) (width 0.5) (layer "F.Cu") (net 2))
 (segment (start 135.382 114.808) (end 135.382 111.154) (width 0.5) (layer "F.Cu") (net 17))
 (segment (start 136.034 115.46) (end 135.382 114.808) (width 0.5) (layer "F.Cu") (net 17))
 (segment (start 138.4705 115.46) (end 136.034 115.46) (width 0.5) (layer "F.Cu") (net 17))
 (segment (start 140.1045 117.094) (end 138.4705 115.46) (width 0.5) (layer "F.Cu") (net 17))
 (segment (start 142.748 120.337949) (end 142.748 119.438051) (width 0.5) (layer "F.Cu") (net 17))
 (segment (start 142.748 119.438051) (end 140.403949 117.094) (width 0.5) (layer "F.Cu") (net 17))
 (segment (start 140.403949 117.094) (end 140.1045 117.094) (width 0.5) (layer "F.Cu") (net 17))
 (segment (start 140.657949 122.428) (end 142.748 120.337949) (width 0.5) (layer "F.Cu") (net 17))
 (segment (start 140.6125 122.428) (end 140.657949 122.428) (width 0.5) (layer "F.Cu") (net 17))
 (segment (start 128.524 112.776) (end 128.524 115.6735) (width 0.5) (layer "F.Cu") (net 13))
 (segment (start 128.524 115.6735) (end 128.27 115.9275) (width 0.5) (layer "F.Cu") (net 13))
 (segment (start 130.81 115.9275) (end 128.27 115.9275) (width 0.5) (layer "F.Cu") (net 13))
 (segment (start 129.032 111.154) (end 128.935 111.251) (width 0.5) (layer "F.Cu") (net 13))
 (segment (start 128.935 111.251) (end 128.935 112.365) (width 0.5) (layer "F.Cu") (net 13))
 (segment (start 128.935 112.365) (end 128.524 112.776) (width 0.5) (layer "F.Cu") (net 13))
 (segment (start 136.652 90.678) (end 136.398 90.424) (width 0.5) (layer "F.Cu") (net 10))
 (segment (start 136.398 90.424) (end 136.398 88.9) (width 0.5) (layer "F.Cu") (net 10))
 (segment (start 136.652 101.854) (end 136.652 90.678) (width 0.5) (layer "F.Cu") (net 10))
 (segment (start 135.583 101.653) (end 135.583 90.625) (width 0.5) (layer "F.Cu") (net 11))
 (segment (start 135.382 101.854) (end 135.583 101.653) (width 0.5) (layer "F.Cu") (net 11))
 (segment (start 135.583 90.625) (end 133.858 88.9) (width 0.5) (layer "F.Cu") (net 11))
 (segment (start 133.096 95.447949) (end 133.604 94.939949) (width 0.5) (layer "F.Cu") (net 12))
 (segment (start 131.572 101.854) (end 131.572 100.840949) (width 0.5) (layer "F.Cu") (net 12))
 (segment (start 131.572 100.840949) (end 133.096 99.316949) (width 0.5) (layer "F.Cu") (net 12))
 (segment (start 133.604 94.939949) (end 133.604 91.186) (width 0.5) (layer "F.Cu") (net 12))
 (segment (start 133.604 91.186) (end 131.318 88.9) (width 0.5) (layer "F.Cu") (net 12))
 (segment (start 133.096 99.316949) (end 133.096 95.447949) (width 0.5) (layer "F.Cu") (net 12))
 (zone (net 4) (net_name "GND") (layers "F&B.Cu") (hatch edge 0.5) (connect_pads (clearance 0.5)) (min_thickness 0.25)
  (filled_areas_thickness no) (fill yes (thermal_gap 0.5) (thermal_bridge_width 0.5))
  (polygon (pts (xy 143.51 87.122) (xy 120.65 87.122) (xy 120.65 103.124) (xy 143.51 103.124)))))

